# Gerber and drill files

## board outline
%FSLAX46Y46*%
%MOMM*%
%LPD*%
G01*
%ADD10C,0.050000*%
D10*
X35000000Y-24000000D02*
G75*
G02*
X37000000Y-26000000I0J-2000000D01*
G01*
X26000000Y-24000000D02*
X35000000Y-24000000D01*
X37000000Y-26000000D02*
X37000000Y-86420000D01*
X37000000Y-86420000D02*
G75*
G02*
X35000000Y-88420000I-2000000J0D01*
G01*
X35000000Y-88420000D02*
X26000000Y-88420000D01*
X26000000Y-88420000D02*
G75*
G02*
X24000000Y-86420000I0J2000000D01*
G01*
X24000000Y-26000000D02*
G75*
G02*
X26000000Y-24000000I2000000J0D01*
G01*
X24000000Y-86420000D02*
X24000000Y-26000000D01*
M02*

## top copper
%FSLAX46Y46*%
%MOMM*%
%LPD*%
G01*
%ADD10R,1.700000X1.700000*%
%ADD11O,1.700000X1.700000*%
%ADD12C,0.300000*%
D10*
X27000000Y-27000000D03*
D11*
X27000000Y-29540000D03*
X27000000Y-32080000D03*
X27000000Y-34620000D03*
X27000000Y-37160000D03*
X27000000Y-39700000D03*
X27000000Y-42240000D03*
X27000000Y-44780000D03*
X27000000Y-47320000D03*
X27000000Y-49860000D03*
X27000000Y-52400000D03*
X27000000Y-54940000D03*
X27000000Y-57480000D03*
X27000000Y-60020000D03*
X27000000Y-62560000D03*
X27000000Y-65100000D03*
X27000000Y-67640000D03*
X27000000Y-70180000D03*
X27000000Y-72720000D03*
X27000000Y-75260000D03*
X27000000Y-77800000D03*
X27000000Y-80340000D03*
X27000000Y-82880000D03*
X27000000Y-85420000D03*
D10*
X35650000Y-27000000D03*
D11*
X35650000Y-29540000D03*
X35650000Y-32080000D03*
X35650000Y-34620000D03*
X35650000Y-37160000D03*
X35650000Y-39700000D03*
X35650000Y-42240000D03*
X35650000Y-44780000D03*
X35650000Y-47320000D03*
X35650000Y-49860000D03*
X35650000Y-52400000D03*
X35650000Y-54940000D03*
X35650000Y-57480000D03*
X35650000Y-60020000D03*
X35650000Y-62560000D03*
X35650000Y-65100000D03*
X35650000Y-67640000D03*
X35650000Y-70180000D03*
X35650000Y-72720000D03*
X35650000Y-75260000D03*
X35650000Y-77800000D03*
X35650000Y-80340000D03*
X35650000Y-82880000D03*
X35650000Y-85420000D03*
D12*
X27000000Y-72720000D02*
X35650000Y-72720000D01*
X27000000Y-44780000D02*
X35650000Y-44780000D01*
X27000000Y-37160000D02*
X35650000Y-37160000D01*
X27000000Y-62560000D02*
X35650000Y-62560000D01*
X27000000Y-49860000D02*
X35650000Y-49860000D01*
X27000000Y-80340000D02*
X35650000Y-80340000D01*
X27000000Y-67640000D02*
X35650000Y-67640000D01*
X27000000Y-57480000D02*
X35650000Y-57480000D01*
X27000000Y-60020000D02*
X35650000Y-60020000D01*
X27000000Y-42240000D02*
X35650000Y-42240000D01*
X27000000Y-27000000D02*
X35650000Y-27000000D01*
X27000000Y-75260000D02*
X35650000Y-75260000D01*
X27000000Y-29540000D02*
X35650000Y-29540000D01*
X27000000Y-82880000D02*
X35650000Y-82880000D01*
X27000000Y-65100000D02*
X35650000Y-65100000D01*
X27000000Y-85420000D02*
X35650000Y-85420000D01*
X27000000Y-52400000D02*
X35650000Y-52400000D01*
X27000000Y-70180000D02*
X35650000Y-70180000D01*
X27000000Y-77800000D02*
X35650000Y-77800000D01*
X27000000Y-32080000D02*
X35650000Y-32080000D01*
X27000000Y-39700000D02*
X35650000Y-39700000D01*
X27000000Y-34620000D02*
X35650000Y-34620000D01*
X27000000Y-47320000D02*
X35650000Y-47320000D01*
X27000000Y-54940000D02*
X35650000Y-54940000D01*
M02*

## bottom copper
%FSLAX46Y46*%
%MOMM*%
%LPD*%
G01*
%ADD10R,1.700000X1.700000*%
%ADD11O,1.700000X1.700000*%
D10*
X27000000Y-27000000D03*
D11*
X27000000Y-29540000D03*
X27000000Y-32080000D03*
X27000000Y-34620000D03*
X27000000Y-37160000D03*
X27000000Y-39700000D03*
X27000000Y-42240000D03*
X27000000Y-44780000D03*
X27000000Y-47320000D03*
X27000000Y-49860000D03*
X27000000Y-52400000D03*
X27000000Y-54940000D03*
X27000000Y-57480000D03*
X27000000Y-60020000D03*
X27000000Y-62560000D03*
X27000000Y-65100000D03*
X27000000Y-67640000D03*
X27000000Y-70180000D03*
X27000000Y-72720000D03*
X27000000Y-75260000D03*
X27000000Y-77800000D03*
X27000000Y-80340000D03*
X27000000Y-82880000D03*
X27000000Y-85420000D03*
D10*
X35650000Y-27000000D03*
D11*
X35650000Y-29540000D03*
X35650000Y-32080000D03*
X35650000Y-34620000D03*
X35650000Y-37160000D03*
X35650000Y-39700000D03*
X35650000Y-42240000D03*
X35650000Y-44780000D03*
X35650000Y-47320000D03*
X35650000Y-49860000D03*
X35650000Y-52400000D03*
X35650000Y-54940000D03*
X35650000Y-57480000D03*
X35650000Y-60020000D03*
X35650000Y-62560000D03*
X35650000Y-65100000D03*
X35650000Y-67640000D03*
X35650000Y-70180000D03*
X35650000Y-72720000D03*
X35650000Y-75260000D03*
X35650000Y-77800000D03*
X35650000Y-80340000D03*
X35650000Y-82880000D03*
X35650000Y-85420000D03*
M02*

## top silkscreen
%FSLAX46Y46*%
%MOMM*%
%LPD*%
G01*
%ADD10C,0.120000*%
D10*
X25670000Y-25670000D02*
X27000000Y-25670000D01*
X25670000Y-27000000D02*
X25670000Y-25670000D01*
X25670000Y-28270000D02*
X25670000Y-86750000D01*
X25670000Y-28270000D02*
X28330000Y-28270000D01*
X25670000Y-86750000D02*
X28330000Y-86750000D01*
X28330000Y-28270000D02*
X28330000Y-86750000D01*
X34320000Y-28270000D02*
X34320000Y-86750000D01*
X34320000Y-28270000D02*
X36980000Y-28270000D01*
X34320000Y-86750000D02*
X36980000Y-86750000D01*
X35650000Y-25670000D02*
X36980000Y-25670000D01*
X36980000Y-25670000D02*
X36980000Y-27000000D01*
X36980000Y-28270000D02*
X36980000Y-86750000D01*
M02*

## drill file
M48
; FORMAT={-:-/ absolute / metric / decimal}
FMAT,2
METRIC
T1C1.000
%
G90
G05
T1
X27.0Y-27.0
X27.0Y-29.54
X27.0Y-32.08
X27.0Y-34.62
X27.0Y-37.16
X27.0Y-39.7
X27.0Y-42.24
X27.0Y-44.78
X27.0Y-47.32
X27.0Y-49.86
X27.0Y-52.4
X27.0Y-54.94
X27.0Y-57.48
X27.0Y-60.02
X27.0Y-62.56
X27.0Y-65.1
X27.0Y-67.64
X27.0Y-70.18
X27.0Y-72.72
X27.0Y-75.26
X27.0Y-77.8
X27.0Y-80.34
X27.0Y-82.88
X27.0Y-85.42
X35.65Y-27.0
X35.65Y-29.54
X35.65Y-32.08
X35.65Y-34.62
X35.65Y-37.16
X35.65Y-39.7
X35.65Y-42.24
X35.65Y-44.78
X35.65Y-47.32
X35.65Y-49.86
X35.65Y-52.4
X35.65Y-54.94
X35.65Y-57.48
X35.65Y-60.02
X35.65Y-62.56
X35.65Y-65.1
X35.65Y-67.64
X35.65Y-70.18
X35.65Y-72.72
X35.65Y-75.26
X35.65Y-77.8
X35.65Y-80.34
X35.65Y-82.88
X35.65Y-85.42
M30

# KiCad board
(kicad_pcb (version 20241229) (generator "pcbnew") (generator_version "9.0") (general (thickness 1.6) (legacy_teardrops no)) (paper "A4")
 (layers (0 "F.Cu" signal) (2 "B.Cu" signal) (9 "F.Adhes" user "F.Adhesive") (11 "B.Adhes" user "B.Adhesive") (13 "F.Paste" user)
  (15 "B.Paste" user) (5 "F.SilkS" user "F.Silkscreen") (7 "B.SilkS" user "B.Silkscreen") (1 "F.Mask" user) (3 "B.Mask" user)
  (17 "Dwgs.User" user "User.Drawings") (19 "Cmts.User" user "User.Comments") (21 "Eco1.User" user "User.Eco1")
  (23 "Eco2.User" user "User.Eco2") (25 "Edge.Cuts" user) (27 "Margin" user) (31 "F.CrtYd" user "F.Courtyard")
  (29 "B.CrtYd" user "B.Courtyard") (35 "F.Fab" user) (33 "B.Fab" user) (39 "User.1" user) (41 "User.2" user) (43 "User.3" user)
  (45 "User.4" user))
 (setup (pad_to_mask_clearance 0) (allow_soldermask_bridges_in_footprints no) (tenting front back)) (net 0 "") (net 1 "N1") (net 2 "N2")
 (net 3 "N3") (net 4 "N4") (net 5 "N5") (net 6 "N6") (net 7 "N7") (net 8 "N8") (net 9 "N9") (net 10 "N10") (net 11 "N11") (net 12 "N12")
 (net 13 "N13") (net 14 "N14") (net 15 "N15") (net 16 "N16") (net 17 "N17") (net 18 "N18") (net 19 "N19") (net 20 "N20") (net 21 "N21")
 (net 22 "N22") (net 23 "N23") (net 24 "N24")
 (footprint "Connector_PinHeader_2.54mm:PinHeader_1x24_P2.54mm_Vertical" (layer "F.Cu") (at 27 27)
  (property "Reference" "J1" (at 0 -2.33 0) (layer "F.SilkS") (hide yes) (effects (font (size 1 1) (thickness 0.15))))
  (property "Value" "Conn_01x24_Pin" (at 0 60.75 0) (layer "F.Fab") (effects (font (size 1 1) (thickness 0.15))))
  (fp_line (start -1.33 -1.33) (end 0 -1.33) (stroke (width 0.12) (type solid)) (layer "F.SilkS"))
  (fp_line (start -1.33 0) (end -1.33 -1.33) (stroke (width 0.12) (type solid)) (layer "F.SilkS"))
  (fp_line (start -1.33 1.27) (end -1.33 59.75) (stroke (width 0.12) (type solid)) (layer "F.SilkS"))
  (fp_line (start -1.33 1.27) (end 1.33 1.27) (stroke (width 0.12) (type solid)) (layer "F.SilkS"))
  (fp_line (start -1.33 59.75) (end 1.33 59.75) (stroke (width 0.12) (type solid)) (layer "F.SilkS"))
  (fp_line (start 1.33 1.27) (end 1.33 59.75) (stroke (width 0.12) (type solid)) (layer "F.SilkS"))
  (pad "1" thru_hole rect (at 0 0) (size 1.7 1.7) (drill 1) (layers "*.Cu" "*.Mask") (remove_unused_layers no) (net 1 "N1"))
  (pad "2" thru_hole oval (at 0 2.54) (size 1.7 1.7) (drill 1) (layers "*.Cu" "*.Mask") (remove_unused_layers no) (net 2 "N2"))
  (pad "3" thru_hole oval (at 0 5.08) (size 1.7 1.7) (drill 1) (layers "*.Cu" "*.Mask") (remove_unused_layers no) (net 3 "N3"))
  (pad "4" thru_hole oval (at 0 7.62) (size 1.7 1.7) (drill 1) (layers "*.Cu" "*.Mask") (remove_unused_layers no) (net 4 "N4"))
  (pad "5" thru_hole oval (at 0 10.16) (size 1.7 1.7) (drill 1) (layers "*.Cu" "*.Mask") (remove_unused_layers no) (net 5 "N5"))
  (pad "6" thru_hole oval (at 0 12.7) (size 1.7 1.7) (drill 1) (layers "*.Cu" "*.Mask") (remove_unused_layers no) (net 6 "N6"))
  (pad "7" thru_hole oval (at 0 15.24) (size 1.7 1.7) (drill 1) (layers "*.Cu" "*.Mask") (remove_unused_layers no) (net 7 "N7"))
  (pad "8" thru_hole oval (at 0 17.78) (size 1.7 1.7) (drill 1) (layers "*.Cu" "*.Mask") (remove_unused_layers no) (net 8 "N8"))
  (pad "9" thru_hole oval (at 0 20.32) (size 1.7 1.7) (drill 1) (layers "*.Cu" "*.Mask") (remove_unused_layers no) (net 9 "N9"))
  (pad "10" thru_hole oval (at 0 22.86) (size 1.7 1.7) (drill 1) (layers "*.Cu" "*.Mask") (remove_unused_layers no) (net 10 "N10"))
  (pad "11" thru_hole oval (at 0 25.4) (size 1.7 1.7) (drill 1) (layers "*.Cu" "*.Mask") (remove_unused_layers no) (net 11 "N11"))
  (pad "12" thru_hole oval (at 0 27.94) (size 1.7 1.7) (drill 1) (layers "*.Cu" "*.Mask") (remove_unused_layers no) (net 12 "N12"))
  (pad "13" thru_hole oval (at 0 30.48) (size 1.7 1.7) (drill 1) (layers "*.Cu" "*.Mask") (remove_unused_layers no) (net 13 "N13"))
  (pad "14" thru_hole oval (at 0 33.02) (size 1.7 1.7) (drill 1) (layers "*.Cu" "*.Mask") (remove_unused_layers no) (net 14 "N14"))
  (pad "15" thru_hole oval (at 0 35.56) (size 1.7 1.7) (drill 1) (layers "*.Cu" "*.Mask") (remove_unused_layers no) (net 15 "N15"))
  (pad "16" thru_hole oval (at 0 38.1) (size 1.7 1.7) (drill 1) (layers "*.Cu" "*.Mask") (remove_unused_layers no) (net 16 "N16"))
  (pad "17" thru_hole oval (at 0 40.64) (size 1.7 1.7) (drill 1) (layers "*.Cu" "*.Mask") (remove_unused_layers no) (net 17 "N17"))
  (pad "18" thru_hole oval (at 0 43.18) (size 1.7 1.7) (drill 1) (layers "*.Cu" "*.Mask") (remove_unused_layers no) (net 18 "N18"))
  (pad "19" thru_hole oval (at 0 45.72) (size 1.7 1.7) (drill 1) (layers "*.Cu" "*.Mask") (remove_unused_layers no) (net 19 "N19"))
  (pad "20" thru_hole oval (at 0 48.26) (size 1.7 1.7) (drill 1) (layers "*.Cu" "*.Mask") (remove_unused_layers no) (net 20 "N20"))
  (pad "21" thru_hole oval (at 0 50.8) (size 1.7 1.7) (drill 1) (layers "*.Cu" "*.Mask") (remove_unused_layers no) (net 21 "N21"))
  (pad "22" thru_hole oval (at 0 53.34) (size 1.7 1.7) (drill 1) (layers "*.Cu" "*.Mask") (remove_unused_layers no) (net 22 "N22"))
  (pad "23" thru_hole oval (at 0 55.88) (size 1.7 1.7) (drill 1) (layers "*.Cu" "*.Mask") (remove_unused_layers no) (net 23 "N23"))
  (pad "24" thru_hole oval (at 0 58.42) (size 1.7 1.7) (drill 1) (layers "*.Cu" "*.Mask") (remove_unused_layers no) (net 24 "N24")))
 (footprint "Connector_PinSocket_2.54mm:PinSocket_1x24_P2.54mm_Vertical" (layer "F.Cu") (at 35.65 27)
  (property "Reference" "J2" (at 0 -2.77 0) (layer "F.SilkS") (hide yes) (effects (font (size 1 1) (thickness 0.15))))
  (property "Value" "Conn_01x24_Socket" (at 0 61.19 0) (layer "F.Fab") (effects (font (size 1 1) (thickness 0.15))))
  (fp_line (start -1.33 1.27) (end -1.33 59.75) (stroke (width 0.12) (type solid)) (layer "F.SilkS"))
  (fp_line (start -1.33 1.27) (end 1.33 1.27) (stroke (width 0.12) (type solid)) (layer "F.SilkS"))
  (fp_line (start -1.33 59.75) (end 1.33 59.75) (stroke (width 0.12) (type solid)) (layer "F.SilkS"))
  (fp_line (start 0 -1.33) (end 1.33 -1.33) (stroke (width 0.12) (type solid)) (layer "F.SilkS"))
  (fp_line (start 1.33 -1.33) (end 1.33 0) (stroke (width 0.12) (type solid)) (layer "F.SilkS"))
  (fp_line (start 1.33 1.27) (end 1.33 59.75) (stroke (width 0.12) (type solid)) (layer "F.SilkS"))
  (pad "1" thru_hole rect (at 0 0) (size 1.7 1.7) (drill 1) (layers "*.Cu" "*.Mask") (remove_unused_layers no) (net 1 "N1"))
  (pad "2" thru_hole oval (at 0 2.54) (size 1.7 1.7) (drill 1) (layers "*.Cu" "*.Mask") (remove_unused_layers no) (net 2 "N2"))
  (pad "3" thru_hole oval (at 0 5.08) (size 1.7 1.7) (drill 1) (layers "*.Cu" "*.Mask") (remove_unused_layers no) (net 3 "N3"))
  (pad "4" thru_hole oval (at 0 7.62) (size 1.7 1.7) (drill 1) (layers "*.Cu" "*.Mask") (remove_unused_layers no) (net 4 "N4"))
  (pad "5" thru_hole oval (at 0 10.16) (size 1.7 1.7) (drill 1) (layers "*.Cu" "*.Mask") (remove_unused_layers no) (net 5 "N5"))
  (pad "6" thru_hole oval (at 0 12.7) (size 1.7 1.7) (drill 1) (layers "*.Cu" "*.Mask") (remove_unused_layers no) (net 6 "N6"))
  (pad "7" thru_hole oval (at 0 15.24) (size 1.7 1.7) (drill 1) (layers "*.Cu" "*.Mask") (remove_unused_layers no) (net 7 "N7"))
  (pad "8" thru_hole oval (at 0 17.78) (size 1.7 1.7) (drill 1) (layers "*.Cu" "*.Mask") (remove_unused_layers no) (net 8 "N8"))
  (pad "9" thru_hole oval (at 0 20.32) (size 1.7 1.7) (drill 1) (layers "*.Cu" "*.Mask") (remove_unused_layers no) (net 9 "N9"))
  (pad "10" thru_hole oval (at 0 22.86) (size 1.7 1.7) (drill 1) (layers "*.Cu" "*.Mask") (remove_unused_layers no) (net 10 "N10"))
  (pad "11" thru_hole oval (at 0 25.4) (size 1.7 1.7) (drill 1) (layers "*.Cu" "*.Mask") (remove_unused_layers no) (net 11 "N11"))
  (pad "12" thru_hole oval (at 0 27.94) (size 1.7 1.7) (drill 1) (layers "*.Cu" "*.Mask") (remove_unused_layers no) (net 12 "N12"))
  (pad "13" thru_hole oval (at 0 30.48) (size 1.7 1.7) (drill 1) (layers "*.Cu" "*.Mask") (remove_unused_layers no) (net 13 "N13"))
  (pad "14" thru_hole oval (at 0 33.02) (size 1.7 1.7) (drill 1) (layers "*.Cu" "*.Mask") (remove_unused_layers no) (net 14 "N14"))
  (pad "15" thru_hole oval (at 0 35.56) (size 1.7 1.7) (drill 1) (layers "*.Cu" "*.Mask") (remove_unused_layers no) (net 15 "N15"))
  (pad "16" thru_hole oval (at 0 38.1) (size 1.7 1.7) (drill 1) (layers "*.Cu" "*.Mask") (remove_unused_layers no) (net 16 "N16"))
  (pad "17" thru_hole oval (at 0 40.64) (size 1.7 1.7) (drill 1) (layers "*.Cu" "*.Mask") (remove_unused_layers no) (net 17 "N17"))
  (pad "18" thru_hole oval (at 0 43.18) (size 1.7 1.7) (drill 1) (layers "*.Cu" "*.Mask") (remove_unused_layers no) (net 18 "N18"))
  (pad "19" thru_hole oval (at 0 45.72) (size 1.7 1.7) (drill 1) (layers "*.Cu" "*.Mask") (remove_unused_layers no) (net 19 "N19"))
  (pad "20" thru_hole oval (at 0 48.26) (size 1.7 1.7) (drill 1) (layers "*.Cu" "*.Mask") (remove_unused_layers no) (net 20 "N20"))
  (pad "21" thru_hole oval (at 0 50.8) (size 1.7 1.7) (drill 1) (layers "*.Cu" "*.Mask") (remove_unused_layers no) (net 21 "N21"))
  (pad "22" thru_hole oval (at 0 53.34) (size 1.7 1.7) (drill 1) (layers "*.Cu" "*.Mask") (remove_unused_layers no) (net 22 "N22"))
  (pad "23" thru_hole oval (at 0 55.88) (size 1.7 1.7) (drill 1) (layers "*.Cu" "*.Mask") (remove_unused_layers no) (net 23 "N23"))
  (pad "24" thru_hole oval (at 0 58.42) (size 1.7 1.7) (drill 1) (layers "*.Cu" "*.Mask") (remove_unused_layers no) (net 24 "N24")))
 (gr_arc (start 35 24) (mid 36.414214 24.585786) (end 37 26) (stroke (width 0.05) (type default)) (layer "Edge.Cuts"))
 (gr_line (start 26 24) (end 35 24) (stroke (width 0.05) (type default)) (layer "Edge.Cuts"))
 (gr_line (start 37 26) (end 37 86.42) (stroke (width 0.05) (type default)) (layer "Edge.Cuts"))
 (gr_arc (start 37 86.42) (mid 36.414214 87.834214) (end 35 88.42) (stroke (width 0.05) (type default)) (layer "Edge.Cuts"))
 (gr_line (start 35 88.42) (end 26 88.42) (stroke (width 0.05) (type default)) (layer "Edge.Cuts"))
 (gr_arc (start 26 88.42) (mid 24.585786 87.834214) (end 24 86.42) (stroke (width 0.05) (type default)) (layer "Edge.Cuts"))
 (gr_arc (start 24 26) (mid 24.585786 24.585786) (end 26 24) (stroke (width 0.05) (type default)) (layer "Edge.Cuts"))
 (gr_line (start 24 86.42) (end 24 26) (stroke (width 0.05) (type default)) (layer "Edge.Cuts"))
 (segment (start 27 72.72) (end 35.65 72.72) (width 0.3) (layer "F.Cu") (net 19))
 (segment (start 27 44.78) (end 35.65 44.78) (width 0.3) (layer "F.Cu") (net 8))
 (segment (start 27 37.16) (end 35.65 37.16) (width 0.3) (layer "F.Cu") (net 5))
 (segment (start 27 62.56) (end 35.65 62.56) (width 0.3) (layer "F.Cu") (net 15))
 (segment (start 27 49.86) (end 35.65 49.86) (width 0.3) (layer "F.Cu") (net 10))
 (segment (start 27 80.34) (end 35.65 80.34) (width 0.3) (layer "F.Cu") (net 22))
 (segment (start 27 67.64) (end 35.65 67.64) (width 0.3) (layer "F.Cu") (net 17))
 (segment (start 27 57.48) (end 35.65 57.48) (width 0.3) (layer "F.Cu") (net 13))
 (segment (start 27 60.02) (end 35.65 60.02) (width 0.3) (layer "F.Cu") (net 14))
 (segment (start 27 42.24) (end 35.65 42.24) (width 0.3) (layer "F.Cu") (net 7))
 (segment (start 27 27) (end 35.65 27) (width 0.3) (layer "F.Cu") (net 1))
 (segment (start 27 75.26) (end 35.65 75.26) (width 0.3) (layer "F.Cu") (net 20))
 (segment (start 27 29.54) (end 35.65 29.54) (width 0.3) (layer "F.Cu") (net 2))
 (segment (start 27 82.88) (end 35.65 82.88) (width 0.3) (layer "F.Cu") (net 23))
 (segment (start 27 65.1) (end 35.65 65.1) (width 0.3) (layer "F.Cu") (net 16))
 (segment (start 27 85.42) (end 35.65 85.42) (width 0.3) (layer "F.Cu") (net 24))
 (segment (start 27 52.4) (end 35.65 52.4) (width 0.3) (layer "F.Cu") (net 11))
 (segment (start 27 70.18) (end 35.65 70.18) (width 0.3) (layer "F.Cu") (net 18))
 (segment (start 27 77.8) (end 35.65 77.8) (width 0.3) (layer "F.Cu") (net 21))
 (segment (start 27 32.08) (end 35.65 32.08) (width 0.3) (layer "F.Cu") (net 3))
 (segment (start 27 39.7) (end 35.65 39.7) (width 0.3) (layer "F.Cu") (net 6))
 (segment (start 27 34.62) (end 35.65 34.62) (width 0.3) (layer "F.Cu") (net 4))
 (segment (start 27 47.32) (end 35.65 47.32) (width 0.3) (layer "F.Cu") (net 9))
 (segment (start 27 54.94) (end 35.65 54.94) (width 0.3) (layer "F.Cu") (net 12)))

